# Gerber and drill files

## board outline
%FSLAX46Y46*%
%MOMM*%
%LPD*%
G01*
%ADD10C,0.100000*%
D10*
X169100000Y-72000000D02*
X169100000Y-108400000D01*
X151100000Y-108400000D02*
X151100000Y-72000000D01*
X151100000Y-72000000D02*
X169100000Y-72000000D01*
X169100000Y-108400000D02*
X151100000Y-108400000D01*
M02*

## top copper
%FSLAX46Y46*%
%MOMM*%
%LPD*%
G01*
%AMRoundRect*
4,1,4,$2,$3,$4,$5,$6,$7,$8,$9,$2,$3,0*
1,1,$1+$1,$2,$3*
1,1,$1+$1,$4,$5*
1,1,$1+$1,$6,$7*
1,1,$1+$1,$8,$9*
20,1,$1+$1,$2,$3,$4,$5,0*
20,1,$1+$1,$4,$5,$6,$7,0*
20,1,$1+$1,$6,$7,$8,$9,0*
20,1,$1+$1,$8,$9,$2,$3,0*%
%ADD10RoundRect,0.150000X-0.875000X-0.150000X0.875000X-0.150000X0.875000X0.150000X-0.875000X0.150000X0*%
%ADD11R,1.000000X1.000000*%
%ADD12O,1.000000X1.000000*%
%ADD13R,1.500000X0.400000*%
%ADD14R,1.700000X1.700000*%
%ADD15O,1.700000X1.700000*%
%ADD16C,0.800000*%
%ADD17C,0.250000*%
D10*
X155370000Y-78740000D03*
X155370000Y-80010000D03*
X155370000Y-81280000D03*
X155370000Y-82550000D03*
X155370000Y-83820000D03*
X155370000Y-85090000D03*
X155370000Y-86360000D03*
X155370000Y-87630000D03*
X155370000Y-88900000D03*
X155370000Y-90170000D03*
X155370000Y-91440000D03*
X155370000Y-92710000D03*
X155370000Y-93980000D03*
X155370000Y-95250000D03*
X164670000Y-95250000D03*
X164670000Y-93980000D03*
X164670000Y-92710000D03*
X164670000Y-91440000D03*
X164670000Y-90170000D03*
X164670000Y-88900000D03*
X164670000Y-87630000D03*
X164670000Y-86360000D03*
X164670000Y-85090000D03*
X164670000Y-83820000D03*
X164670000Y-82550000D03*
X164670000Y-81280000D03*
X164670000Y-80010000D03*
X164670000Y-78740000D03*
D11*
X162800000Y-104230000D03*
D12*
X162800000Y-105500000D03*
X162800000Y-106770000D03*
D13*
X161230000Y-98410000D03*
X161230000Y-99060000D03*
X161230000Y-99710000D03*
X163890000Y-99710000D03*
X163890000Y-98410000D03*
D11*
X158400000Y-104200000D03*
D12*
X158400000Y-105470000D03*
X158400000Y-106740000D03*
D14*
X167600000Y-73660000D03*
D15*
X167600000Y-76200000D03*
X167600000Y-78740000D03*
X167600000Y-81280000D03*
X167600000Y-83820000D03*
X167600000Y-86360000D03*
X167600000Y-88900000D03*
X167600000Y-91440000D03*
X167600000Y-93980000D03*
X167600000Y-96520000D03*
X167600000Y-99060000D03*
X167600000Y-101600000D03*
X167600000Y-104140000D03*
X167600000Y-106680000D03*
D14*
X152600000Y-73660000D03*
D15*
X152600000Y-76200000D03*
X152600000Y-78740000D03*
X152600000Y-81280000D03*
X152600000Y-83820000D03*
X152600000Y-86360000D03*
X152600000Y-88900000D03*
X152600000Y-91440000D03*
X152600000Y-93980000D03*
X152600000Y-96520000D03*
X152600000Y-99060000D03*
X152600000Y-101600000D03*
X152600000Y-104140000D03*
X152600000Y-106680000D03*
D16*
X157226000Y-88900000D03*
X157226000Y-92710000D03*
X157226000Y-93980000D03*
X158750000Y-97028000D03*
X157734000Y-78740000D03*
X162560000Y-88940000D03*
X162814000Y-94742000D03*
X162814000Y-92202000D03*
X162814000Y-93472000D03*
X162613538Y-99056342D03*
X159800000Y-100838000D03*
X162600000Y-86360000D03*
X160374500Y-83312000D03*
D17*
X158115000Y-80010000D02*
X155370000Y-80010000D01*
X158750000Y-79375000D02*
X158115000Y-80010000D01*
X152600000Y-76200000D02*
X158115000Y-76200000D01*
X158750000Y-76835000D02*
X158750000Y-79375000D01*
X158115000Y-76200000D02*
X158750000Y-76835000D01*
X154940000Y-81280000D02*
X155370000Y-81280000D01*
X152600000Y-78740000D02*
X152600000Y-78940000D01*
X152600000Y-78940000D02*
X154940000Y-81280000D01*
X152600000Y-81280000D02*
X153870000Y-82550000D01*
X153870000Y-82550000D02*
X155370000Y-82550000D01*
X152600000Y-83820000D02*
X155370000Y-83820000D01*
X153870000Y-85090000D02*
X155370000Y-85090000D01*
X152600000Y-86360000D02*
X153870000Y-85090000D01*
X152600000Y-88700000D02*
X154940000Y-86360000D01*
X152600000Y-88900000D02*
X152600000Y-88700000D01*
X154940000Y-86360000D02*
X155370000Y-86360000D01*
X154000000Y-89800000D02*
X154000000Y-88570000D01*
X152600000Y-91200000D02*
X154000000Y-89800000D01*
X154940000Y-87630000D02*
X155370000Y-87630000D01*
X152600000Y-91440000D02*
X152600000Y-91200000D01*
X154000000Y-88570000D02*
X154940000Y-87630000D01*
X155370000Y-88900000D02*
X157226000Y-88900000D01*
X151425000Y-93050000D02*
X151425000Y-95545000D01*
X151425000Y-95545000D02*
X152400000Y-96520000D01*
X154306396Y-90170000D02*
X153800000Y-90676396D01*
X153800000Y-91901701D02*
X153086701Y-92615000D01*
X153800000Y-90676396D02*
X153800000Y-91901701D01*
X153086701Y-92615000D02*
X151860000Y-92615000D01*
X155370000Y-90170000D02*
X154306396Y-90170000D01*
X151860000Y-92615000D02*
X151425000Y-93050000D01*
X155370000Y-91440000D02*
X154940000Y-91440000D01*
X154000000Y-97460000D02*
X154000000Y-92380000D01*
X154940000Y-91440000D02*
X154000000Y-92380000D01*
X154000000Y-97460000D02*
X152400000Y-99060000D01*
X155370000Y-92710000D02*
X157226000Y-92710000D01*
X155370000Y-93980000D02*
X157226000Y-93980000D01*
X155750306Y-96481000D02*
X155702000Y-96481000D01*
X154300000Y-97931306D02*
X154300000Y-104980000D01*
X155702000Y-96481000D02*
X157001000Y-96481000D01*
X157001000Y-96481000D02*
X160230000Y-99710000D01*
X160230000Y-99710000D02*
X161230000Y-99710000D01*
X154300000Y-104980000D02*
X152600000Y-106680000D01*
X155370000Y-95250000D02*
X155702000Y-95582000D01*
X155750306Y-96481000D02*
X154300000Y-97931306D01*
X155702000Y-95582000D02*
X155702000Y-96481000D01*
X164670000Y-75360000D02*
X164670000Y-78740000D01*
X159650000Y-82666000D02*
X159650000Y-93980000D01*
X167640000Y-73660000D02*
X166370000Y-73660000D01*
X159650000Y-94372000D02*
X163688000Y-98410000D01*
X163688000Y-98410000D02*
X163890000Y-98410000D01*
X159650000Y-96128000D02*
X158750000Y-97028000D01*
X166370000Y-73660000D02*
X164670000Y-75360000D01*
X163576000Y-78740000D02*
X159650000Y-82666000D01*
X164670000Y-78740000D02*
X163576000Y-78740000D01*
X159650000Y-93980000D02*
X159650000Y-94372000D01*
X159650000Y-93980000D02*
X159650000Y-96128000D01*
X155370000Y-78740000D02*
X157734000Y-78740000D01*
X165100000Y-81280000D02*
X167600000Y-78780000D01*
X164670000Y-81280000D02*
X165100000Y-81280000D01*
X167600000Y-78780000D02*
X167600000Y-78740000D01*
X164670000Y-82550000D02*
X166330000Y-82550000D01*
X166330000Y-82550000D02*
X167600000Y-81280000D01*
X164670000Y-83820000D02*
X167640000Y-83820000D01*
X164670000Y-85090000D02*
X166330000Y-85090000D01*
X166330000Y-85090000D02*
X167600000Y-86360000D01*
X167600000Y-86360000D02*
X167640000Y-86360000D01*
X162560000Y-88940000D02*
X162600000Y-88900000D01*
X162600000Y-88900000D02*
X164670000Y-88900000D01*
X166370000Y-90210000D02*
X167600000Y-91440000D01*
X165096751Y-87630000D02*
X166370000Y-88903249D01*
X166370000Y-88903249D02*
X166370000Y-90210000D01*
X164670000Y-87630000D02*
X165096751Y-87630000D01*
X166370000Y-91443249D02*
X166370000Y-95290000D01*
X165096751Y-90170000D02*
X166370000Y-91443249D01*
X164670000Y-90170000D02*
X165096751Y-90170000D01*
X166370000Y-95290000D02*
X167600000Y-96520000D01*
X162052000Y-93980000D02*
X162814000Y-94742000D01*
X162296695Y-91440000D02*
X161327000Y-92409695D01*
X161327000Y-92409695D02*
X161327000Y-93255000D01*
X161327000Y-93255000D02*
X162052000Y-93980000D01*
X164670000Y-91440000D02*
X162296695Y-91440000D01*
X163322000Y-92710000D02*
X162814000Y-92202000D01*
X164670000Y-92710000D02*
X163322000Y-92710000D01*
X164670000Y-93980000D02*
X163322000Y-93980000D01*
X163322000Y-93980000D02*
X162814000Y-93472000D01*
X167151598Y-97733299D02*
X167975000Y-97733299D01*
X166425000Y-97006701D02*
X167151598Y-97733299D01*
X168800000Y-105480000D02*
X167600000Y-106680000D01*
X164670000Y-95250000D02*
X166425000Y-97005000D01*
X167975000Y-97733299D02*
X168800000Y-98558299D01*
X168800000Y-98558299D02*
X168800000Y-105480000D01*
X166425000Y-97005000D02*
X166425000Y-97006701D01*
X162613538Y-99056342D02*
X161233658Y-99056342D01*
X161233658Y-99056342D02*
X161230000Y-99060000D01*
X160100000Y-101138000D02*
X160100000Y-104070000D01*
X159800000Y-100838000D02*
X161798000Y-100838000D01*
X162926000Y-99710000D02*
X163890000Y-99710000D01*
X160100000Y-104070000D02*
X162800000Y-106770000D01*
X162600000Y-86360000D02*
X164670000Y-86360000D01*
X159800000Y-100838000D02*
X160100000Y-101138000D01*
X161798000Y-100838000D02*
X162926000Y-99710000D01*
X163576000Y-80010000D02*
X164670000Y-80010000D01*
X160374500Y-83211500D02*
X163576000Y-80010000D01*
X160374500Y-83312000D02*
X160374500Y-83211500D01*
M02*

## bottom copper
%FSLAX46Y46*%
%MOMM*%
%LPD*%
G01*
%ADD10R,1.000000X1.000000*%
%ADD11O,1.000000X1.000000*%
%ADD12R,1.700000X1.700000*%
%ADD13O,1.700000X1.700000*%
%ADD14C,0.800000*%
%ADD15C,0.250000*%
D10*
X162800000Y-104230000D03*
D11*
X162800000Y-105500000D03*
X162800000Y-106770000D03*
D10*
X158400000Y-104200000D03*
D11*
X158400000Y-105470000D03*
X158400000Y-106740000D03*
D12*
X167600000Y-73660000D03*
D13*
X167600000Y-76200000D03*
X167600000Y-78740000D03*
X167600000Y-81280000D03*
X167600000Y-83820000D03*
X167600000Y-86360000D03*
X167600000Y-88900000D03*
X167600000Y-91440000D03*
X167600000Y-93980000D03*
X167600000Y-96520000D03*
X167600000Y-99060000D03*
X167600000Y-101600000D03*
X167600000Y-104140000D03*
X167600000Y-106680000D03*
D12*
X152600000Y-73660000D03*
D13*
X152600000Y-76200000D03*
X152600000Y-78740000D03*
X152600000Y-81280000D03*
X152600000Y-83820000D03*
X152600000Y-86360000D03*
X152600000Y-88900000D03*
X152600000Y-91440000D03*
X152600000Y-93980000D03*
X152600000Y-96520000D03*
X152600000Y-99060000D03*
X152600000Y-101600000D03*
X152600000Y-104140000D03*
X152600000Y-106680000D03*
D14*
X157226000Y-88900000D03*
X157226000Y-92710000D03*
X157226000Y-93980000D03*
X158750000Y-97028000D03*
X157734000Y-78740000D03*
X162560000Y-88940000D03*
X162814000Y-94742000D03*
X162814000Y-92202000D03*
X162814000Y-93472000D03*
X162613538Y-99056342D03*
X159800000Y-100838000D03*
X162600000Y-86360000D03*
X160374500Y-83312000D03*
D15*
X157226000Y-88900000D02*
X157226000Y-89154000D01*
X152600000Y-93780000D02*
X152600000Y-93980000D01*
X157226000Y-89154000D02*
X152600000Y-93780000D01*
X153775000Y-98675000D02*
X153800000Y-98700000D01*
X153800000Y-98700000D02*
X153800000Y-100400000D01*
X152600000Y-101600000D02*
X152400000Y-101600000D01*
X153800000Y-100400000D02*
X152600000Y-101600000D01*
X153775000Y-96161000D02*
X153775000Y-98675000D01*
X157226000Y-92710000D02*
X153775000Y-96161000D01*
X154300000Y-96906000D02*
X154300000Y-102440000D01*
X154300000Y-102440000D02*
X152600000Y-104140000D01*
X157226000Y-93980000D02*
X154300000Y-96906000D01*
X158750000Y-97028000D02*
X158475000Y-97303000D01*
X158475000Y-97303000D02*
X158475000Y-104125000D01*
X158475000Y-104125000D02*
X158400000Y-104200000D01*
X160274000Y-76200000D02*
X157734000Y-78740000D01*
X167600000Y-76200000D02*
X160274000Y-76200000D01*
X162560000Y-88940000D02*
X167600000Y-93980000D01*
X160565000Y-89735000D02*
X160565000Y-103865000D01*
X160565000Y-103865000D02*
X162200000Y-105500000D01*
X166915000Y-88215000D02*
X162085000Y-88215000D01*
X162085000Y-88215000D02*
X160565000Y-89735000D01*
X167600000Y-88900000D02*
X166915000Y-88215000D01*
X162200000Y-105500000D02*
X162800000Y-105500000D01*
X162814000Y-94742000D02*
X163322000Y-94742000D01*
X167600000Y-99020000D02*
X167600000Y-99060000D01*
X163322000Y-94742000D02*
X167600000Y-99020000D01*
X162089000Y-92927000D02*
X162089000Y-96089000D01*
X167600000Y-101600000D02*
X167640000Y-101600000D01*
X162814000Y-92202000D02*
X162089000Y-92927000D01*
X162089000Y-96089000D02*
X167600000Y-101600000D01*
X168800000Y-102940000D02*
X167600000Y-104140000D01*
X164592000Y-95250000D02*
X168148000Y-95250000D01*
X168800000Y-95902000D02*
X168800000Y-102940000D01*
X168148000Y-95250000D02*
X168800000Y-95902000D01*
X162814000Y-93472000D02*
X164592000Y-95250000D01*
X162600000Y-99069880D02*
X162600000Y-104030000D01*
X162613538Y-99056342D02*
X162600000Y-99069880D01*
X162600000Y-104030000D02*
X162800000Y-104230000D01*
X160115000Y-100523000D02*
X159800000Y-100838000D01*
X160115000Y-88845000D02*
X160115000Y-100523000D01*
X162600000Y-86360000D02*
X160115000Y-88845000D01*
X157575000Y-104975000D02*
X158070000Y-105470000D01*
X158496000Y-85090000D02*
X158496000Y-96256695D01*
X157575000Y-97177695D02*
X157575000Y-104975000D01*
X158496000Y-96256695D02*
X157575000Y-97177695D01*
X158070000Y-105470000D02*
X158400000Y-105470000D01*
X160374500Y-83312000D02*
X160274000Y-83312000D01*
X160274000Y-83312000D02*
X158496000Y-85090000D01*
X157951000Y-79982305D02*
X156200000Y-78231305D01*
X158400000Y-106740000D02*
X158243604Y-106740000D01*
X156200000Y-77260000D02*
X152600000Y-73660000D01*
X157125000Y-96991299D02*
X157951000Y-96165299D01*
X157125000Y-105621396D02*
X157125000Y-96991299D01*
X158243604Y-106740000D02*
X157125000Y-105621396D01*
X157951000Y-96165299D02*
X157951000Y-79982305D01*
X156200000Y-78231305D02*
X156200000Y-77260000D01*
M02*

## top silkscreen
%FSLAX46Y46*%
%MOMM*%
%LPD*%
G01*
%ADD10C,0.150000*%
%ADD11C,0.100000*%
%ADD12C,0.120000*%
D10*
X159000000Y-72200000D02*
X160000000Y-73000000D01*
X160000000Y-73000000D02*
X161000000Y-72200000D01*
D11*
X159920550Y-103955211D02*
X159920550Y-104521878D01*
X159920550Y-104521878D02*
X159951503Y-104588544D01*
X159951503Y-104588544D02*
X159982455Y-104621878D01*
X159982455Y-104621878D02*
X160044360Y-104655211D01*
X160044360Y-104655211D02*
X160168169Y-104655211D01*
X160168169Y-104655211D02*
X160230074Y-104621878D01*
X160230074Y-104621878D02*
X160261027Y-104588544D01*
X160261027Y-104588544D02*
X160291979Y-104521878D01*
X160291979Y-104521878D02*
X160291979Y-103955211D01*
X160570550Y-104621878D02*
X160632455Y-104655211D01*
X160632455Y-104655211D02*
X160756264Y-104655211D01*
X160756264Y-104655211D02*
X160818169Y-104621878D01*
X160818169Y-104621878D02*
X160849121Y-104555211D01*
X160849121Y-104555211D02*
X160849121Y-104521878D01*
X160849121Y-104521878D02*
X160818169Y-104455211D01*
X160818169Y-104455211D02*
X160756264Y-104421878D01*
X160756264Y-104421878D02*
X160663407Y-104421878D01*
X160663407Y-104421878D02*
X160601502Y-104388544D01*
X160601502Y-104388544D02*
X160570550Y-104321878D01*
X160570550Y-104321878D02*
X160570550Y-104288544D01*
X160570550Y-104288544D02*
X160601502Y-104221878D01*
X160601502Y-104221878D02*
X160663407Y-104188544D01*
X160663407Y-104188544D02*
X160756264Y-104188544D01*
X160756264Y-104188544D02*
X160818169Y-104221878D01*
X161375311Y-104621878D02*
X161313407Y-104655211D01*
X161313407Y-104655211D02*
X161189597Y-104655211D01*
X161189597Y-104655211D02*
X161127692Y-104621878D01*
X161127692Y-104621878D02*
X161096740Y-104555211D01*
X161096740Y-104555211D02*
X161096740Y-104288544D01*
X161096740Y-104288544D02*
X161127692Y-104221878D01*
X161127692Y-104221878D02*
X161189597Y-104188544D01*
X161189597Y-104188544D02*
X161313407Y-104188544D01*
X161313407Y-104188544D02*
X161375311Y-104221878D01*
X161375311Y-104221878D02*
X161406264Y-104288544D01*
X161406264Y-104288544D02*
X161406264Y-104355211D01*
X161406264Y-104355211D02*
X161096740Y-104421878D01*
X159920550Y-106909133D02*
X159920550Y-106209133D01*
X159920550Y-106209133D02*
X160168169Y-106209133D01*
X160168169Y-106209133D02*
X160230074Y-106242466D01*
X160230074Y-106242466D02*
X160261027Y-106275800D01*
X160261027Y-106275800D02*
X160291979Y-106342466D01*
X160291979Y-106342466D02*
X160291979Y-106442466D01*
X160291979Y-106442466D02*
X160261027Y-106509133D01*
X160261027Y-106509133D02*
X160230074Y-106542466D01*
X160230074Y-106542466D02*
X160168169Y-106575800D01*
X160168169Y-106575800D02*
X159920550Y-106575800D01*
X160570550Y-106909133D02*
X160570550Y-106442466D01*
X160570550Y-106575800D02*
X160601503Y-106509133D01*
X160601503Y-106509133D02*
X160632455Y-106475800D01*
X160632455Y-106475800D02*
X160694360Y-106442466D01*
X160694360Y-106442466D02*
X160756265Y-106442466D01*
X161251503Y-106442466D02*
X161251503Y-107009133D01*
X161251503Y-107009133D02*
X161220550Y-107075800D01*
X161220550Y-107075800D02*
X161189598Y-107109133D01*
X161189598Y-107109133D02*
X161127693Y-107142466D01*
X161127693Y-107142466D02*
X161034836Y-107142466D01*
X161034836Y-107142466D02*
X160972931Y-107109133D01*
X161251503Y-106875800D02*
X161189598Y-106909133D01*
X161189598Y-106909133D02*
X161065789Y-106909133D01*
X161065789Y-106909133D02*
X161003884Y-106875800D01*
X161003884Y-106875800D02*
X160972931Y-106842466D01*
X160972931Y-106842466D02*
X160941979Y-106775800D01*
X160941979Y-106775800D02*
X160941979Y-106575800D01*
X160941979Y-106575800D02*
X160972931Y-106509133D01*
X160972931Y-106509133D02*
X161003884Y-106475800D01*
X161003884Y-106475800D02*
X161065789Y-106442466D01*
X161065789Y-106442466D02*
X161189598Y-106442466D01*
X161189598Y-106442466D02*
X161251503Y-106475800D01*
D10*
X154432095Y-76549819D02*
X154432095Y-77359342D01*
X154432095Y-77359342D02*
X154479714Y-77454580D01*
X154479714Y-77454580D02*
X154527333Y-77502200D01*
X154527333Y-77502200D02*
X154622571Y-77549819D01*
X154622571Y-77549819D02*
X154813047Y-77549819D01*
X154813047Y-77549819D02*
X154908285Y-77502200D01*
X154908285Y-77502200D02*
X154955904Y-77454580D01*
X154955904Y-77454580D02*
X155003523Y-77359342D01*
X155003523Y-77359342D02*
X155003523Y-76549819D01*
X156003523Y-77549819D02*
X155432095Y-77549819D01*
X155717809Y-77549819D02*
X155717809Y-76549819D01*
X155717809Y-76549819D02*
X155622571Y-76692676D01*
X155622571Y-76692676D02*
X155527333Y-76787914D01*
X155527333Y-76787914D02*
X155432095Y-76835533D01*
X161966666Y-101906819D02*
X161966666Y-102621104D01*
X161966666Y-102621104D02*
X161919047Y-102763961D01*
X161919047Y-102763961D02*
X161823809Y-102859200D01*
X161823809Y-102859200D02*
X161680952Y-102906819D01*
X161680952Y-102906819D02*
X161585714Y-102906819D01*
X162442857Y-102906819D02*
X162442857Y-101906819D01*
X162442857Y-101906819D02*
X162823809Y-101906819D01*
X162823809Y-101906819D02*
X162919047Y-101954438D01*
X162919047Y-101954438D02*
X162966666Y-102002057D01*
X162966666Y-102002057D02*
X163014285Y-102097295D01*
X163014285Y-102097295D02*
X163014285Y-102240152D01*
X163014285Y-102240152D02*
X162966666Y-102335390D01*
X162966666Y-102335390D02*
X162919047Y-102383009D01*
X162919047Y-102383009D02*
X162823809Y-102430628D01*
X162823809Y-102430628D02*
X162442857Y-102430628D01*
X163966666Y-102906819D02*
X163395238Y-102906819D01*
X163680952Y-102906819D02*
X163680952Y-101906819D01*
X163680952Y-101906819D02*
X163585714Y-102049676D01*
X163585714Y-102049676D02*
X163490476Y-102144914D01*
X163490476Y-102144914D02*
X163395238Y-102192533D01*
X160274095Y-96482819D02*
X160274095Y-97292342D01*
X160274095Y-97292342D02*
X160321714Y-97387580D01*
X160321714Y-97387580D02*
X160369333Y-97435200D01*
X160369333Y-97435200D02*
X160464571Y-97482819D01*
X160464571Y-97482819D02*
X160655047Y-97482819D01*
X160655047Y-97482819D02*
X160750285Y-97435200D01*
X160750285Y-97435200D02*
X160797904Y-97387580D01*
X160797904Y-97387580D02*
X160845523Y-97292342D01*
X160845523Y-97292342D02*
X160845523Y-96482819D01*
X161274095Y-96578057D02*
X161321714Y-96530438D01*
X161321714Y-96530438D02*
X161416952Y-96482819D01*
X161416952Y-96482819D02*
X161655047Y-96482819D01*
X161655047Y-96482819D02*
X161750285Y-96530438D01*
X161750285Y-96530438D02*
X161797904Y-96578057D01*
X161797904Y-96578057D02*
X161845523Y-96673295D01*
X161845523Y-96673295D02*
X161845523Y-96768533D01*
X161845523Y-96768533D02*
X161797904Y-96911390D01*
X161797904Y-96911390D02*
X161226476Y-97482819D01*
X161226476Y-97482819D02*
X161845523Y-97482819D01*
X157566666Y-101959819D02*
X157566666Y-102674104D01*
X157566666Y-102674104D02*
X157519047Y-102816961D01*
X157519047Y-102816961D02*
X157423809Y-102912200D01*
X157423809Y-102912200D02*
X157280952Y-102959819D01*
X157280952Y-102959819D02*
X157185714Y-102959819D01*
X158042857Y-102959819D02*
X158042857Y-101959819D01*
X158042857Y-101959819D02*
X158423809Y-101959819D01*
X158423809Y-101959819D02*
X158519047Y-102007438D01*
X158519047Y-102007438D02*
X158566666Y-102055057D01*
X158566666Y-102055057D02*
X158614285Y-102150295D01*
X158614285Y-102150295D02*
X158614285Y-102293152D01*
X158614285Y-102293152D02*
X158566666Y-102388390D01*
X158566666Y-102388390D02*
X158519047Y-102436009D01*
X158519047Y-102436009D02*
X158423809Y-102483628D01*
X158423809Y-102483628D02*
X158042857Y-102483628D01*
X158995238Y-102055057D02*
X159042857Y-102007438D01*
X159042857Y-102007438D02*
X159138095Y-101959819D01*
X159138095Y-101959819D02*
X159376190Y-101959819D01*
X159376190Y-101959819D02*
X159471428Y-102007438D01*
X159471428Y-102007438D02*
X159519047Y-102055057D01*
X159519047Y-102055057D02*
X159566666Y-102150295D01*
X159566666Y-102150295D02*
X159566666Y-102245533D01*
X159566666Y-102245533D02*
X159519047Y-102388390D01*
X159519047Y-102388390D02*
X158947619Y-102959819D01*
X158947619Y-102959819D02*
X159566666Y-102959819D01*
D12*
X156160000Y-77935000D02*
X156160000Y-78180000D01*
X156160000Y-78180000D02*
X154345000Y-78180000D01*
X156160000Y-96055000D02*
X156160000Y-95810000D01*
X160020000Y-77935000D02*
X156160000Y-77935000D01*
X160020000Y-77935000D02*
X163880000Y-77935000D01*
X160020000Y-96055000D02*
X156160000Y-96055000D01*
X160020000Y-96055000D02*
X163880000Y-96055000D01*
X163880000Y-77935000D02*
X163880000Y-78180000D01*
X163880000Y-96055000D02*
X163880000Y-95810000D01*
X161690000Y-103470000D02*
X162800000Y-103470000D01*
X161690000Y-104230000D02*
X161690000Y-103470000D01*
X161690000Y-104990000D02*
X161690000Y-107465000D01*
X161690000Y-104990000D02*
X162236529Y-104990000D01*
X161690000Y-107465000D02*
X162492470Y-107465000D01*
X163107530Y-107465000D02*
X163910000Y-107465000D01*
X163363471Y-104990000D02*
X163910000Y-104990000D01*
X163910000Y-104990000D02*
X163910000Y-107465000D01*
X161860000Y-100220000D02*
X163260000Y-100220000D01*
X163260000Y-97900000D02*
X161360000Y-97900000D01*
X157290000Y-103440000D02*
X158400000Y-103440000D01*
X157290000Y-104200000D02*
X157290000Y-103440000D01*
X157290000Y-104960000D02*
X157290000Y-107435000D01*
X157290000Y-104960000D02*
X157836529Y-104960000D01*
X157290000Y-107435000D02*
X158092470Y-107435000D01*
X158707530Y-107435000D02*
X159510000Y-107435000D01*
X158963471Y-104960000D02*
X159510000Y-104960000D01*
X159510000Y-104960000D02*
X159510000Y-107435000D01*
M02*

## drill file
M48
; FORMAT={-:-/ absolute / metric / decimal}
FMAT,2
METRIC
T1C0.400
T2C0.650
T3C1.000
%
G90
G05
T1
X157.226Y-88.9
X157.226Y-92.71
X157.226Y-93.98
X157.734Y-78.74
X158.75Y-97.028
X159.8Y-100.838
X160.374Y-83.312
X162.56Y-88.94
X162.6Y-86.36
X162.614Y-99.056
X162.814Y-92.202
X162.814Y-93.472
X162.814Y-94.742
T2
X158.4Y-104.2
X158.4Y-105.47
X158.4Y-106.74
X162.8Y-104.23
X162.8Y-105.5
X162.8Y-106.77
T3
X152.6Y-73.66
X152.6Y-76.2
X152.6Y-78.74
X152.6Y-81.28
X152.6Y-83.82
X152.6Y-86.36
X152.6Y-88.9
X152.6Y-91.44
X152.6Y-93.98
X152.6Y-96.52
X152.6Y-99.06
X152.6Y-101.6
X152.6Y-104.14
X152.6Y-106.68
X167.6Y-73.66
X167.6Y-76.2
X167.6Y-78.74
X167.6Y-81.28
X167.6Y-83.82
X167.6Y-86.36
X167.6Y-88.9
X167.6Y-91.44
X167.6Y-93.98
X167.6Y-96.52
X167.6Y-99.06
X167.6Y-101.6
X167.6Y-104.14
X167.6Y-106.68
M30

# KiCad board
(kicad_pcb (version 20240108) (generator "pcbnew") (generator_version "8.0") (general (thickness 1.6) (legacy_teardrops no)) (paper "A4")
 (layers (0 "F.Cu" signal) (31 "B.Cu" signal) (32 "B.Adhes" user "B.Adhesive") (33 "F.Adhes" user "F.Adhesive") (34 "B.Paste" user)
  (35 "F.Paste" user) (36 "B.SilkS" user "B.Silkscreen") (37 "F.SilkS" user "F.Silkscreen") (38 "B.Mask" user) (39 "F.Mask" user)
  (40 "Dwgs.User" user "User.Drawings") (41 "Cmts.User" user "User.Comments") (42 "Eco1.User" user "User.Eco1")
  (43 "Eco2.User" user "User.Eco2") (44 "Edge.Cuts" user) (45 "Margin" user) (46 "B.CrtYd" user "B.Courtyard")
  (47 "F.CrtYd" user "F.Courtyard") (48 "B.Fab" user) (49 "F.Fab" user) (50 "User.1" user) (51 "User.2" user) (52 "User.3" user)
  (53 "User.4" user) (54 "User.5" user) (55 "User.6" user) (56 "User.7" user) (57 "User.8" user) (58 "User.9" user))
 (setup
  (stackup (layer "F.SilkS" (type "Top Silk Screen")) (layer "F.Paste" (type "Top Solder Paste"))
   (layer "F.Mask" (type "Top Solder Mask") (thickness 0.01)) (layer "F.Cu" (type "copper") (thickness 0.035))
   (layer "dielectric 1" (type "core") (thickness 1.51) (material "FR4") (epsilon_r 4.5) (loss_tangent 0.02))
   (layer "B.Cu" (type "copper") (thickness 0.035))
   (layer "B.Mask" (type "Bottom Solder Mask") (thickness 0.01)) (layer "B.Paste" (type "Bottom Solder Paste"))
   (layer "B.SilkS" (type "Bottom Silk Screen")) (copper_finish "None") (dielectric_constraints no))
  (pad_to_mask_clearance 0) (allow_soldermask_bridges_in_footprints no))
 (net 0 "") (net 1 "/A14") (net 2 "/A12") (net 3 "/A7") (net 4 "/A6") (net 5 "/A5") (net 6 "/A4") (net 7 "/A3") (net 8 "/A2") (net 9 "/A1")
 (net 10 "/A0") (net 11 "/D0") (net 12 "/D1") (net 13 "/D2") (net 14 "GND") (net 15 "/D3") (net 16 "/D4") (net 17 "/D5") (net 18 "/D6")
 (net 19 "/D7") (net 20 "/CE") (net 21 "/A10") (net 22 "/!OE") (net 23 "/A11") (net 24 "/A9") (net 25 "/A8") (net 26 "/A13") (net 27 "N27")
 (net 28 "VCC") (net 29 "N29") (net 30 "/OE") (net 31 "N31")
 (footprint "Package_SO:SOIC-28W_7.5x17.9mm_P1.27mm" (layer "F.Cu") (at 160.02 86.995)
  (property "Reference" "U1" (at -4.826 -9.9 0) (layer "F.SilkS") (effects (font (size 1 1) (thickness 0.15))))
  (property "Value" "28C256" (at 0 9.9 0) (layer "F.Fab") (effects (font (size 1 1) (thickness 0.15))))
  (fp_line (start -3.86 -9.06) (end -3.86 -8.815) (stroke (width 0.12) (type solid)) (layer "F.SilkS"))
  (fp_line (start -3.86 -8.815) (end -5.675 -8.815) (stroke (width 0.12) (type solid)) (layer "F.SilkS"))
  (fp_line (start -3.86 9.06) (end -3.86 8.815) (stroke (width 0.12) (type solid)) (layer "F.SilkS"))
  (fp_line (start 0 -9.06) (end -3.86 -9.06) (stroke (width 0.12) (type solid)) (layer "F.SilkS"))
  (fp_line (start 0 -9.06) (end 3.86 -9.06) (stroke (width 0.12) (type solid)) (layer "F.SilkS"))
  (fp_line (start 0 9.06) (end -3.86 9.06) (stroke (width 0.12) (type solid)) (layer "F.SilkS"))
  (fp_line (start 0 9.06) (end 3.86 9.06) (stroke (width 0.12) (type solid)) (layer "F.SilkS"))
  (fp_line (start 3.86 -9.06) (end 3.86 -8.815) (stroke (width 0.12) (type solid)) (layer "F.SilkS"))
  (fp_line (start 3.86 9.06) (end 3.86 8.815) (stroke (width 0.12) (type solid)) (layer "F.SilkS"))
  (pad "1" smd roundrect (at -4.65 -8.255) (size 2.05 0.6) (layers "F.Cu" "F.Paste" "F.Mask") (roundrect_rratio 0.25) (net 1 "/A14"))
  (pad "2" smd roundrect (at -4.65 -6.985) (size 2.05 0.6) (layers "F.Cu" "F.Paste" "F.Mask") (roundrect_rratio 0.25) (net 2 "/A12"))
  (pad "3" smd roundrect (at -4.65 -5.715) (size 2.05 0.6) (layers "F.Cu" "F.Paste" "F.Mask") (roundrect_rratio 0.25) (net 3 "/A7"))
  (pad "4" smd roundrect (at -4.65 -4.445) (size 2.05 0.6) (layers "F.Cu" "F.Paste" "F.Mask") (roundrect_rratio 0.25) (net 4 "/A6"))
  (pad "5" smd roundrect (at -4.65 -3.175) (size 2.05 0.6) (layers "F.Cu" "F.Paste" "F.Mask") (roundrect_rratio 0.25) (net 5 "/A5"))
  (pad "6" smd roundrect (at -4.65 -1.905) (size 2.05 0.6) (layers "F.Cu" "F.Paste" "F.Mask") (roundrect_rratio 0.25) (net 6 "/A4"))
  (pad "7" smd roundrect (at -4.65 -0.635) (size 2.05 0.6) (layers "F.Cu" "F.Paste" "F.Mask") (roundrect_rratio 0.25) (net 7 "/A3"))
  (pad "8" smd roundrect (at -4.65 0.635) (size 2.05 0.6) (layers "F.Cu" "F.Paste" "F.Mask") (roundrect_rratio 0.25) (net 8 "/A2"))
  (pad "9" smd roundrect (at -4.65 1.905) (size 2.05 0.6) (layers "F.Cu" "F.Paste" "F.Mask") (roundrect_rratio 0.25) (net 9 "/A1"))
  (pad "10" smd roundrect (at -4.65 3.175) (size 2.05 0.6) (layers "F.Cu" "F.Paste" "F.Mask") (roundrect_rratio 0.25) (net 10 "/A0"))
  (pad "11" smd roundrect (at -4.65 4.445) (size 2.05 0.6) (layers "F.Cu" "F.Paste" "F.Mask") (roundrect_rratio 0.25) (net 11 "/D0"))
  (pad "12" smd roundrect (at -4.65 5.715) (size 2.05 0.6) (layers "F.Cu" "F.Paste" "F.Mask") (roundrect_rratio 0.25) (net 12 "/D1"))
  (pad "13" smd roundrect (at -4.65 6.985) (size 2.05 0.6) (layers "F.Cu" "F.Paste" "F.Mask") (roundrect_rratio 0.25) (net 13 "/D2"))
  (pad "14" smd roundrect (at -4.65 8.255) (size 2.05 0.6) (layers "F.Cu" "F.Paste" "F.Mask") (roundrect_rratio 0.25) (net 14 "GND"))
  (pad "15" smd roundrect (at 4.65 8.255) (size 2.05 0.6) (layers "F.Cu" "F.Paste" "F.Mask") (roundrect_rratio 0.25) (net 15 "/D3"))
  (pad "16" smd roundrect (at 4.65 6.985) (size 2.05 0.6) (layers "F.Cu" "F.Paste" "F.Mask") (roundrect_rratio 0.25) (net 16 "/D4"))
  (pad "17" smd roundrect (at 4.65 5.715) (size 2.05 0.6) (layers "F.Cu" "F.Paste" "F.Mask") (roundrect_rratio 0.25) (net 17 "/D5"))
  (pad "18" smd roundrect (at 4.65 4.445) (size 2.05 0.6) (layers "F.Cu" "F.Paste" "F.Mask") (roundrect_rratio 0.25) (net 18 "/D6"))
  (pad "19" smd roundrect (at 4.65 3.175) (size 2.05 0.6) (layers "F.Cu" "F.Paste" "F.Mask") (roundrect_rratio 0.25) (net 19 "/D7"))
  (pad "20" smd roundrect (at 4.65 1.905) (size 2.05 0.6) (layers "F.Cu" "F.Paste" "F.Mask") (roundrect_rratio 0.25) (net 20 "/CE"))
  (pad "21" smd roundrect (at 4.65 0.635) (size 2.05 0.6) (layers "F.Cu" "F.Paste" "F.Mask") (roundrect_rratio 0.25) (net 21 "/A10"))
  (pad "22" smd roundrect (at 4.65 -0.635) (size 2.05 0.6) (layers "F.Cu" "F.Paste" "F.Mask") (roundrect_rratio 0.25) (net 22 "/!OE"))
  (pad "23" smd roundrect (at 4.65 -1.905) (size 2.05 0.6) (layers "F.Cu" "F.Paste" "F.Mask") (roundrect_rratio 0.25) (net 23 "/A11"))
  (pad "24" smd roundrect (at 4.65 -3.175) (size 2.05 0.6) (layers "F.Cu" "F.Paste" "F.Mask") (roundrect_rratio 0.25) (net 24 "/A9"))
  (pad "25" smd roundrect (at 4.65 -4.445) (size 2.05 0.6) (layers "F.Cu" "F.Paste" "F.Mask") (roundrect_rratio 0.25) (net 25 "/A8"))
  (pad "26" smd roundrect (at 4.65 -5.715) (size 2.05 0.6) (layers "F.Cu" "F.Paste" "F.Mask") (roundrect_rratio 0.25) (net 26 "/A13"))
  (pad "27" smd roundrect (at 4.65 -6.985) (size 2.05 0.6) (layers "F.Cu" "F.Paste" "F.Mask") (roundrect_rratio 0.25) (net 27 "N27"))
  (pad "28" smd roundrect (at 4.65 -8.255) (size 2.05 0.6) (layers "F.Cu" "F.Paste" "F.Mask") (roundrect_rratio 0.25) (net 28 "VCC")))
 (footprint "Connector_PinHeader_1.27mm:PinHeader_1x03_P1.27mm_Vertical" (layer "F.Cu") (at 162.8 104.23)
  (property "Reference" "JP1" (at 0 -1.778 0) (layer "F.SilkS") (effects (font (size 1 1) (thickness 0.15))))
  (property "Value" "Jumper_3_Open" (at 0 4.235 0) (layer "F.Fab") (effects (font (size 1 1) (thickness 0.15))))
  (fp_line (start -1.11 -0.76) (end 0 -0.76) (stroke (width 0.12) (type solid)) (layer "F.SilkS"))
  (fp_line (start -1.11 0) (end -1.11 -0.76) (stroke (width 0.12) (type solid)) (layer "F.SilkS"))
  (fp_line (start -1.11 0.76) (end -1.11 3.235) (stroke (width 0.12) (type solid)) (layer "F.SilkS"))
  (fp_line (start -1.11 0.76) (end -0.563471 0.76) (stroke (width 0.12) (type solid)) (layer "F.SilkS"))
  (fp_line (start -1.11 3.235) (end -0.30753 3.235) (stroke (width 0.12) (type solid)) (layer "F.SilkS"))
  (fp_line (start 0.30753 3.235) (end 1.11 3.235) (stroke (width 0.12) (type solid)) (layer "F.SilkS"))
  (fp_line (start 0.563471 0.76) (end 1.11 0.76) (stroke (width 0.12) (type solid)) (layer "F.SilkS"))
  (fp_line (start 1.11 0.76) (end 1.11 3.235) (stroke (width 0.12) (type solid)) (layer "F.SilkS"))
  (pad "1" thru_hole rect (at 0 0) (size 1 1) (drill 0.65) (layers "*.Cu" "*.Mask") (remove_unused_layers no) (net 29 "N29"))
  (pad "2" thru_hole oval (at 0 1.27) (size 1 1) (drill 0.65) (layers "*.Cu" "*.Mask") (remove_unused_layers no) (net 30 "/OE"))
  (pad "3" thru_hole oval (at 0 2.54) (size 1 1) (drill 0.65) (layers "*.Cu" "*.Mask") (remove_unused_layers no) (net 22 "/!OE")))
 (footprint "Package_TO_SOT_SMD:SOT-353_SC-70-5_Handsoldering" (layer "F.Cu") (at 162.56 99.06)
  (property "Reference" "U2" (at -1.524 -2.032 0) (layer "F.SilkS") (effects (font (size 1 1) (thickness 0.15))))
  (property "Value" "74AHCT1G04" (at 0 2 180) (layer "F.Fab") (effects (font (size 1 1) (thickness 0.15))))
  (fp_line (start -0.7 1.16) (end 0.7 1.16) (stroke (width 0.12) (type solid)) (layer "F.SilkS"))
  (fp_line (start 0.7 -1.16) (end -1.2 -1.16) (stroke (width 0.12) (type solid)) (layer "F.SilkS"))
  (pad "1" smd rect (at -1.33 -0.65) (size 1.5 0.4) (layers "F.Cu" "F.Paste" "F.Mask"))
  (pad "2" smd rect (at -1.33 0) (size 1.5 0.4) (layers "F.Cu" "F.Paste" "F.Mask") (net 29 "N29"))
  (pad "3" smd rect (at -1.33 0.65) (size 1.5 0.4) (layers "F.Cu" "F.Paste" "F.Mask") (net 14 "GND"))
  (pad "4" smd rect (at 1.33 0.65) (size 1.5 0.4) (layers "F.Cu" "F.Paste" "F.Mask") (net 22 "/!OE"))
  (pad "5" smd rect (at 1.33 -0.65) (size 1.5 0.4) (layers "F.Cu" "F.Paste" "F.Mask") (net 28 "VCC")))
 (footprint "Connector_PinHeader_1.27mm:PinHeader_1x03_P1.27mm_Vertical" (layer "F.Cu") (at 158.4 104.2)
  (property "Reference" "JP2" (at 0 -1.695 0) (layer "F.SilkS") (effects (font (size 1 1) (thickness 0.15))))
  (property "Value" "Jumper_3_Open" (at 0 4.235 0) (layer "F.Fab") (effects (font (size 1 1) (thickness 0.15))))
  (fp_line (start -1.11 -0.76) (end 0 -0.76) (stroke (width 0.12) (type solid)) (layer "F.SilkS"))
  (fp_line (start -1.11 0) (end -1.11 -0.76) (stroke (width 0.12) (type solid)) (layer "F.SilkS"))
  (fp_line (start -1.11 0.76) (end -1.11 3.235) (stroke (width 0.12) (type solid)) (layer "F.SilkS"))
  (fp_line (start -1.11 0.76) (end -0.563471 0.76) (stroke (width 0.12) (type solid)) (layer "F.SilkS"))
  (fp_line (start -1.11 3.235) (end -0.30753 3.235) (stroke (width 0.12) (type solid)) (layer "F.SilkS"))
  (fp_line (start 0.30753 3.235) (end 1.11 3.235) (stroke (width 0.12) (type solid)) (layer "F.SilkS"))
  (fp_line (start 0.563471 0.76) (end 1.11 0.76) (stroke (width 0.12) (type solid)) (layer "F.SilkS"))
  (fp_line (start 1.11 0.76) (end 1.11 3.235) (stroke (width 0.12) (type solid)) (layer "F.SilkS"))
  (pad "1" thru_hole rect (at 0 0) (size 1 1) (drill 0.65) (layers "*.Cu" "*.Mask") (remove_unused_layers no) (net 28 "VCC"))
  (pad "2" thru_hole oval (at 0 1.27) (size 1 1) (drill 0.65) (layers "*.Cu" "*.Mask") (remove_unused_layers no) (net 27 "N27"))
  (pad "3" thru_hole oval (at 0 2.54) (size 1 1) (drill 0.65) (layers "*.Cu" "*.Mask") (remove_unused_layers no) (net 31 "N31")))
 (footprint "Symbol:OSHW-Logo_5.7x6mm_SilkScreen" (layer "B.Cu") (at 159.893 77.336 180)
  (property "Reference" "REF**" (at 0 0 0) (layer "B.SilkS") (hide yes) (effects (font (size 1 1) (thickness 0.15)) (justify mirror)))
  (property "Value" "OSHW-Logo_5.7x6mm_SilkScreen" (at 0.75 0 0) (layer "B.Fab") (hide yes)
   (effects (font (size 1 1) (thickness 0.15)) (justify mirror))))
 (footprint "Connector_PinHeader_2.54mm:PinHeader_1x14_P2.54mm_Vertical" (layer "B.Cu") (at 167.6 73.66 180)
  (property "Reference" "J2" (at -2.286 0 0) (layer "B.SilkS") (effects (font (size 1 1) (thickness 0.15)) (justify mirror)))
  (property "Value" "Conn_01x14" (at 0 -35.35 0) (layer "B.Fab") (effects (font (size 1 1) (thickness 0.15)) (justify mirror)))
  (pad "1" thru_hole rect (at 0 0 180) (size 1.7 1.7) (drill 1) (layers "*.Cu" "*.Mask") (remove_unused_layers no) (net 28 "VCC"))
  (pad "2" thru_hole oval (at 0 -2.54 180) (size 1.7 1.7) (drill 1) (layers "*.Cu" "*.Mask") (remove_unused_layers no) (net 1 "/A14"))
  (pad "3" thru_hole oval (at 0 -5.08 180) (size 1.7 1.7) (drill 1) (layers "*.Cu" "*.Mask") (remove_unused_layers no) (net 26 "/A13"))
  (pad "4" thru_hole oval (at 0 -7.62 180) (size 1.7 1.7) (drill 1) (layers "*.Cu" "*.Mask") (remove_unused_layers no) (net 25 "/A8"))
  (pad "5" thru_hole oval (at 0 -10.16 180) (size 1.7 1.7) (drill 1) (layers "*.Cu" "*.Mask") (remove_unused_layers no) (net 24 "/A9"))
  (pad "6" thru_hole oval (at 0 -12.7 180) (size 1.7 1.7) (drill 1) (layers "*.Cu" "*.Mask") (remove_unused_layers no) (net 23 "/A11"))
  (pad "7" thru_hole oval (at 0 -15.24 180) (size 1.7 1.7) (drill 1) (layers "*.Cu" "*.Mask") (remove_unused_layers no) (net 30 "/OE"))
  (pad "8" thru_hole oval (at 0 -17.78 180) (size 1.7 1.7) (drill 1) (layers "*.Cu" "*.Mask") (remove_unused_layers no) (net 21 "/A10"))
  (pad "9" thru_hole oval (at 0 -20.32 180) (size 1.7 1.7) (drill 1) (layers "*.Cu" "*.Mask") (remove_unused_layers no) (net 20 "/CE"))
  (pad "10" thru_hole oval (at 0 -22.86 180) (size 1.7 1.7) (drill 1) (layers "*.Cu" "*.Mask") (remove_unused_layers no) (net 19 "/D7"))
  (pad "11" thru_hole oval (at 0 -25.4 180) (size 1.7 1.7) (drill 1) (layers "*.Cu" "*.Mask") (remove_unused_layers no) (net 18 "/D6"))
  (pad "12" thru_hole oval (at 0 -27.94 180) (size 1.7 1.7) (drill 1) (layers "*.Cu" "*.Mask") (remove_unused_layers no) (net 17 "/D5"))
  (pad "13" thru_hole oval (at 0 -30.48 180) (size 1.7 1.7) (drill 1) (layers "*.Cu" "*.Mask") (remove_unused_layers no) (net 16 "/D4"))
  (pad "14" thru_hole oval (at 0 -33.02 180) (size 1.7 1.7) (drill 1) (layers "*.Cu" "*.Mask") (remove_unused_layers no) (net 15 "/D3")))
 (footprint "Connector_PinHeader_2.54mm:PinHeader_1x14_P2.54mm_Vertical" (layer "B.Cu") (at 152.6 73.66 180)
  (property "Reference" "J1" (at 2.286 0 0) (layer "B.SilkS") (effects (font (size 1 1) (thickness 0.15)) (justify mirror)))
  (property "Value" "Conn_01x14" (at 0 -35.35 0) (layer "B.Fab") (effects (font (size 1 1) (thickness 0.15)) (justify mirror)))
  (pad "1" thru_hole rect (at 0 0 180) (size 1.7 1.7) (drill 1) (layers "*.Cu" "*.Mask") (remove_unused_layers no) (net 31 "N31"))
  (pad "2" thru_hole oval (at 0 -2.54 180) (size 1.7 1.7) (drill 1) (layers "*.Cu" "*.Mask") (remove_unused_layers no) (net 2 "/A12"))
  (pad "3" thru_hole oval (at 0 -5.08 180) (size 1.7 1.7) (drill 1) (layers "*.Cu" "*.Mask") (remove_unused_layers no) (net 3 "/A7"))
  (pad "4" thru_hole oval (at 0 -7.62 180) (size 1.7 1.7) (drill 1) (layers "*.Cu" "*.Mask") (remove_unused_layers no) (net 4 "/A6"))
  (pad "5" thru_hole oval (at 0 -10.16 180) (size 1.7 1.7) (drill 1) (layers "*.Cu" "*.Mask") (remove_unused_layers no) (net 5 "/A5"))
  (pad "6" thru_hole oval (at 0 -12.7 180) (size 1.7 1.7) (drill 1) (layers "*.Cu" "*.Mask") (remove_unused_layers no) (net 6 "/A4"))
  (pad "7" thru_hole oval (at 0 -15.24 180) (size 1.7 1.7) (drill 1) (layers "*.Cu" "*.Mask") (remove_unused_layers no) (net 7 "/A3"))
  (pad "8" thru_hole oval (at 0 -17.78 180) (size 1.7 1.7) (drill 1) (layers "*.Cu" "*.Mask") (remove_unused_layers no) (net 8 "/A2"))
  (pad "9" thru_hole oval (at 0 -20.32 180) (size 1.7 1.7) (drill 1) (layers "*.Cu" "*.Mask") (remove_unused_layers no) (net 9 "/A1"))
  (pad "10" thru_hole oval (at 0 -22.86 180) (size 1.7 1.7) (drill 1) (layers "*.Cu" "*.Mask") (remove_unused_layers no) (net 10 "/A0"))
  (pad "11" thru_hole oval (at 0 -25.4 180) (size 1.7 1.7) (drill 1) (layers "*.Cu" "*.Mask") (remove_unused_layers no) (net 11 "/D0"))
  (pad "12" thru_hole oval (at 0 -27.94 180) (size 1.7 1.7) (drill 1) (layers "*.Cu" "*.Mask") (remove_unused_layers no) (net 12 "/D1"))
  (pad "13" thru_hole oval (at 0 -30.48 180) (size 1.7 1.7) (drill 1) (layers "*.Cu" "*.Mask") (remove_unused_layers no) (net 13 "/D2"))
  (pad "14" thru_hole oval (at 0 -33.02 180) (size 1.7 1.7) (drill 1) (layers "*.Cu" "*.Mask") (remove_unused_layers no) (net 14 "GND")))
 (gr_line (start 159 72.2) (end 160 73) (stroke (width 0.15) (type default)) (layer "F.SilkS"))
 (gr_line (start 160 73) (end 161 72.2) (stroke (width 0.15) (type default)) (layer "F.SilkS"))
 (gr_line (start 169.1 72) (end 169.1 108.4) (stroke (width 0.1) (type default)) (layer "Edge.Cuts"))
 (gr_line (start 151.1 108.4) (end 151.1 72) (stroke (width 0.1) (type default)) (layer "Edge.Cuts"))
 (gr_line (start 151.1 72) (end 169.1 72) (stroke (width 0.1) (type default)) (layer "Edge.Cuts"))
 (gr_line (start 169.1 108.4) (end 151.1 108.4) (stroke (width 0.1) (type default)) (layer "Edge.Cuts"))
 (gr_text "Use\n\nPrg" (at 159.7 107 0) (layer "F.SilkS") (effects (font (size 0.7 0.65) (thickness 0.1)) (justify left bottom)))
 (segment (start 158.115 80.01) (end 155.37 80.01) (width 0.25) (layer "F.Cu") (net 2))
 (segment (start 158.75 79.375) (end 158.115 80.01) (width 0.25) (layer "F.Cu") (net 2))
 (segment (start 152.6 76.2) (end 158.115 76.2) (width 0.25) (layer "F.Cu") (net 2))
 (segment (start 158.75 76.835) (end 158.75 79.375) (width 0.25) (layer "F.Cu") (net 2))
 (segment (start 158.115 76.2) (end 158.75 76.835) (width 0.25) (layer "F.Cu") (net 2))
 (segment (start 154.94 81.28) (end 155.37 81.28) (width 0.25) (layer "F.Cu") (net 3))
 (segment (start 152.6 78.74) (end 152.6 78.94) (width 0.25) (layer "F.Cu") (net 3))
 (segment (start 152.6 78.94) (end 154.94 81.28) (width 0.25) (layer "F.Cu") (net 3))
 (segment (start 152.6 81.28) (end 153.87 82.55) (width 0.25) (layer "F.Cu") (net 4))
 (segment (start 153.87 82.55) (end 155.37 82.55) (width 0.25) (layer "F.Cu") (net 4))
 (segment (start 152.6 83.82) (end 155.37 83.82) (width 0.25) (layer "F.Cu") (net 5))
 (segment (start 153.87 85.09) (end 155.37 85.09) (width 0.25) (layer "F.Cu") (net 6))
 (segment (start 152.6 86.36) (end 153.87 85.09) (width 0.25) (layer "F.Cu") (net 6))
 (segment (start 152.6 88.7) (end 154.94 86.36) (width 0.25) (layer "F.Cu") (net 7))
 (segment (start 152.6 88.9) (end 152.6 88.7) (width 0.25) (layer "F.Cu") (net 7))
 (segment (start 154.94 86.36) (end 155.37 86.36) (width 0.25) (layer "F.Cu") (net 7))
 (segment (start 154 89.8) (end 154 88.57) (width 0.25) (layer "F.Cu") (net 8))
 (segment (start 152.6 91.2) (end 154 89.8) (width 0.25) (layer "F.Cu") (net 8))
 (segment (start 154.94 87.63) (end 155.37 87.63) (width 0.25) (layer "F.Cu") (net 8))
 (segment (start 152.6 91.44) (end 152.6 91.2) (width 0.25) (layer "F.Cu") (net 8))
 (segment (start 154 88.57) (end 154.94 87.63) (width 0.25) (layer "F.Cu") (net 8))
 (segment (start 155.37 88.9) (end 157.226 88.9) (width 0.25) (layer "F.Cu") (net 9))
 (via (at 157.226 88.9) (size 0.8) (drill 0.4) (layers "F.Cu" "B.Cu") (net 9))
 (segment (start 157.226 88.9) (end 157.226 89.154) (width 0.25) (layer "B.Cu") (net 9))
 (segment (start 152.6 93.78) (end 152.6 93.98) (width 0.25) (layer "B.Cu") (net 9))
 (segment (start 157.226 89.154) (end 152.6 93.78) (width 0.25) (layer "B.Cu") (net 9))
 (segment (start 151.425 93.05) (end 151.425 95.545) (width 0.25) (layer "F.Cu") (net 10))
 (segment (start 151.425 95.545) (end 152.4 96.52) (width 0.25) (layer "F.Cu") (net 10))
 (segment (start 154.306396 90.17) (end 153.8 90.676396) (width 0.25) (layer "F.Cu") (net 10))
 (segment (start 153.8 91.901701) (end 153.086701 92.615) (width 0.25) (layer "F.Cu") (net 10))
 (segment (start 153.8 90.676396) (end 153.8 91.901701) (width 0.25) (layer "F.Cu") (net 10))
 (segment (start 153.086701 92.615) (end 151.86 92.615) (width 0.25) (layer "F.Cu") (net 10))
 (segment (start 155.37 90.17) (end 154.306396 90.17) (width 0.25) (layer "F.Cu") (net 10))
 (segment (start 151.86 92.615) (end 151.425 93.05) (width 0.25) (layer "F.Cu") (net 10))
 (segment (start 155.37 91.44) (end 154.94 91.44) (width 0.25) (layer "F.Cu") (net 11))
 (segment (start 154 97.46) (end 154 92.38) (width 0.25) (layer "F.Cu") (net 11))
 (segment (start 154.94 91.44) (end 154 92.38) (width 0.25) (layer "F.Cu") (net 11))
 (segment (start 154 97.46) (end 152.4 99.06) (width 0.25) (layer "F.Cu") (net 11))
 (segment (start 155.37 92.71) (end 157.226 92.71) (width 0.25) (layer "F.Cu") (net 12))
 (via (at 157.226 92.71) (size 0.8) (drill 0.4) (layers "F.Cu" "B.Cu") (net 12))
 (segment (start 153.775 98.675) (end 153.8 98.7) (width 0.25) (layer "B.Cu") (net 12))
 (segment (start 153.8 98.7) (end 153.8 100.4) (width 0.25) (layer "B.Cu") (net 12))
 (segment (start 152.6 101.6) (end 152.4 101.6) (width 0.25) (layer "B.Cu") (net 12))
 (segment (start 153.8 100.4) (end 152.6 101.6) (width 0.25) (layer "B.Cu") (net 12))
 (segment (start 153.775 96.161) (end 153.775 98.675) (width 0.25) (layer "B.Cu") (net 12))
 (segment (start 157.226 92.71) (end 153.775 96.161) (width 0.25) (layer "B.Cu") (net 12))
 (segment (start 155.37 93.98) (end 157.226 93.98) (width 0.25) (layer "F.Cu") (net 13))
 (via (at 157.226 93.98) (size 0.8) (drill 0.4) (layers "F.Cu" "B.Cu") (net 13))
 (segment (start 154.3 96.906) (end 154.3 102.44) (width 0.25) (layer "B.Cu") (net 13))
 (segment (start 154.3 102.44) (end 152.6 104.14) (width 0.25) (layer "B.Cu") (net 13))
 (segment (start 157.226 93.98) (end 154.3 96.906) (width 0.25) (layer "B.Cu") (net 13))
 (segment (start 155.750306 96.481) (end 155.702 96.481) (width 0.25) (layer "F.Cu") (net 14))
 (segment (start 154.3 97.931306) (end 154.3 104.98) (width 0.25) (layer "F.Cu") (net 14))
 (segment (start 155.702 96.481) (end 157.001 96.481) (width 0.25) (layer "F.Cu") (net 14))
 (segment (start 157.001 96.481) (end 160.23 99.71) (width 0.25) (layer "F.Cu") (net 14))
 (segment (start 160.23 99.71) (end 161.23 99.71) (width 0.25) (layer "F.Cu") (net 14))
 (segment (start 154.3 104.98) (end 152.6 106.68) (width 0.25) (layer "F.Cu") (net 14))
 (segment (start 155.37 95.25) (end 155.702 95.582) (width 0.25) (layer "F.Cu") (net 14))
 (segment (start 155.750306 96.481) (end 154.3 97.931306) (width 0.25) (layer "F.Cu") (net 14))
 (segment (start 155.702 95.582) (end 155.702 96.481) (width 0.25) (layer "F.Cu") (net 14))
 (segment (start 164.67 75.36) (end 164.67 78.74) (width 0.25) (layer "F.Cu") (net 28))
 (segment (start 159.65 82.666) (end 159.65 93.98) (width 0.25) (layer "F.Cu") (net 28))
 (segment (start 167.64 73.66) (end 166.37 73.66) (width 0.25) (layer "F.Cu") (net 28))
 (segment (start 159.65 94.372) (end 163.688 98.41) (width 0.25) (layer "F.Cu") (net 28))
 (segment (start 163.688 98.41) (end 163.89 98.41) (width 0.25) (layer "F.Cu") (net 28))
 (segment (start 159.65 96.128) (end 158.75 97.028) (width 0.25) (layer "F.Cu") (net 28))
 (segment (start 166.37 73.66) (end 164.67 75.36) (width 0.25) (layer "F.Cu") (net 28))
 (segment (start 163.576 78.74) (end 159.65 82.666) (width 0.25) (layer "F.Cu") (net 28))
 (segment (start 164.67 78.74) (end 163.576 78.74) (width 0.25) (layer "F.Cu") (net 28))
 (segment (start 159.65 93.98) (end 159.65 94.372) (width 0.25) (layer "F.Cu") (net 28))
 (segment (start 159.65 93.98) (end 159.65 96.128) (width 0.25) (layer "F.Cu") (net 28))
 (via (at 158.75 97.028) (size 0.8) (drill 0.4) (layers "F.Cu" "B.Cu") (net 28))
 (segment (start 158.75 97.028) (end 158.475 97.303) (width 0.25) (layer "B.Cu") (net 28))
 (segment (start 158.475 97.303) (end 158.475 104.125) (width 0.25) (layer "B.Cu") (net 28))
 (segment (start 158.475 104.125) (end 158.4 104.2) (width 0.25) (layer "B.Cu") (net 28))
 (segment (start 155.37 78.74) (end 157.734 78.74) (width 0.25) (layer "F.Cu") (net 1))
 (via (at 157.734 78.74) (size 0.8) (drill 0.4) (layers "F.Cu" "B.Cu") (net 1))
 (segment (start 160.274 76.2) (end 157.734 78.74) (width 0.25) (layer "B.Cu") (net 1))
 (segment (start 167.6 76.2) (end 160.274 76.2) (width 0.25) (layer "B.Cu") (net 1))
 (segment (start 165.1 81.28) (end 167.6 78.78) (width 0.25) (layer "F.Cu") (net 26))
 (segment (start 164.67 81.28) (end 165.1 81.28) (width 0.25) (layer "F.Cu") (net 26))
 (segment (start 167.6 78.78) (end 167.6 78.74) (width 0.25) (layer "F.Cu") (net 26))
 (segment (start 164.67 82.55) (end 166.33 82.55) (width 0.25) (layer "F.Cu") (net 25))
 (segment (start 166.33 82.55) (end 167.6 81.28) (width 0.25) (layer "F.Cu") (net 25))
 (segment (start 164.67 83.82) (end 167.64 83.82) (width 0.25) (layer "F.Cu") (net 24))
 (segment (start 164.67 85.09) (end 166.33 85.09) (width 0.25) (layer "F.Cu") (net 23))
 (segment (start 166.33 85.09) (end 167.6 86.36) (width 0.25) (layer "F.Cu") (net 23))
 (segment (start 167.6 86.36) (end 167.64 86.36) (width 0.25) (layer "F.Cu") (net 23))
 (segment (start 162.56 88.94) (end 162.6 88.9) (width 0.25) (layer "F.Cu") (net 20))
 (segment (start 162.6 88.9) (end 164.67 88.9) (width 0.25) (layer "F.Cu") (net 20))
 (via (at 162.56 88.94) (size 0.8) (drill 0.4) (layers "F.Cu" "B.Cu") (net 20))
 (segment (start 162.56 88.94) (end 167.6 93.98) (width 0.25) (layer "B.Cu") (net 20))
 (segment (start 166.37 90.21) (end 167.6 91.44) (width 0.25) (layer "F.Cu") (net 21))
 (segment (start 165.096751 87.63) (end 166.37 88.903249) (width 0.25) (layer "F.Cu") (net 21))
 (segment (start 166.37 88.903249) (end 166.37 90.21) (width 0.25) (layer "F.Cu") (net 21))
 (segment (start 164.67 87.63) (end 165.096751 87.63) (width 0.25) (layer "F.Cu") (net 21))
 (segment (start 160.565 89.735) (end 160.565 103.865) (width 0.25) (layer "B.Cu") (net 30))
 (segment (start 160.565 103.865) (end 162.2 105.5) (width 0.25) (layer "B.Cu") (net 30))
 (segment (start 166.915 88.215) (end 162.085 88.215) (width 0.25) (layer "B.Cu") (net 30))
 (segment (start 162.085 88.215) (end 160.565 89.735) (width 0.25) (layer "B.Cu") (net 30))
 (segment (start 167.6 88.9) (end 166.915 88.215) (width 0.25) (layer "B.Cu") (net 30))
 (segment (start 162.2 105.5) (end 162.8 105.5) (width 0.25) (layer "B.Cu") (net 30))
 (segment (start 166.37 91.443249) (end 166.37 95.29) (width 0.25) (layer "F.Cu") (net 19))
 (segment (start 165.096751 90.17) (end 166.37 91.443249) (width 0.25) (layer "F.Cu") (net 19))
 (segment (start 164.67 90.17) (end 165.096751 90.17) (width 0.25) (layer "F.Cu") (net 19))
 (segment (start 166.37 95.29) (end 167.6 96.52) (width 0.25) (layer "F.Cu") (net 19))
 (segment (start 162.052 93.98) (end 162.814 94.742) (width 0.25) (layer "F.Cu") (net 18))
 (segment (start 162.296695 91.44) (end 161.327 92.409695) (width 0.25) (layer "F.Cu") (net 18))
 (segment (start 161.327 92.409695) (end 161.327 93.255) (width 0.25) (layer "F.Cu") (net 18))
 (segment (start 161.327 93.255) (end 162.052 93.98) (width 0.25) (layer "F.Cu") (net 18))
 (segment (start 164.67 91.44) (end 162.296695 91.44) (width 0.25) (layer "F.Cu") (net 18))
 (via (at 162.814 94.742) (size 0.8) (drill 0.4) (layers "F.Cu" "B.Cu") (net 18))
 (segment (start 162.814 94.742) (end 163.322 94.742) (width 0.25) (layer "B.Cu") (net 18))
 (segment (start 167.6 99.02) (end 167.6 99.06) (width 0.25) (layer "B.Cu") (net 18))
 (segment (start 163.322 94.742) (end 167.6 99.02) (width 0.25) (layer "B.Cu") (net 18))
 (segment (start 163.322 92.71) (end 162.814 92.202) (width 0.25) (layer "F.Cu") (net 17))
 (segment (start 164.67 92.71) (end 163.322 92.71) (width 0.25) (layer "F.Cu") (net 17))
 (via (at 162.814 92.202) (size 0.8) (drill 0.4) (layers "F.Cu" "B.Cu") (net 17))
 (segment (start 162.089 92.927) (end 162.089 96.089) (width 0.25) (layer "B.Cu") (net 17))
 (segment (start 167.6 101.6) (end 167.64 101.6) (width 0.25) (layer "B.Cu") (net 17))
 (segment (start 162.814 92.202) (end 162.089 92.927) (width 0.25) (layer "B.Cu") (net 17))
 (segment (start 162.089 96.089) (end 167.6 101.6) (width 0.25) (layer "B.Cu") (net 17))
 (segment (start 164.67 93.98) (end 163.322 93.98) (width 0.25) (layer "F.Cu") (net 16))
 (segment (start 163.322 93.98) (end 162.814 93.472) (width 0.25) (layer "F.Cu") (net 16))
 (via (at 162.814 93.472) (size 0.8) (drill 0.4) (layers "F.Cu" "B.Cu") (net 16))
 (segment (start 168.8 102.94) (end 167.6 104.14) (width 0.25) (layer "B.Cu") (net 16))
 (segment (start 164.592 95.25) (end 168.148 95.25) (width 0.25) (layer "B.Cu") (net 16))
 (segment (start 168.8 95.902) (end 168.8 102.94) (width 0.25) (layer "B.Cu") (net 16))
 (segment (start 168.148 95.25) (end 168.8 95.902) (width 0.25) (layer "B.Cu") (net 16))
 (segment (start 162.814 93.472) (end 164.592 95.25) (width 0.25) (layer "B.Cu") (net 16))
 (segment (start 167.151598 97.733299) (end 167.975 97.733299) (width 0.25) (layer "F.Cu") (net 15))
 (segment (start 166.425 97.006701) (end 167.151598 97.733299) (width 0.25) (layer "F.Cu") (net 15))
 (segment (start 168.8 105.48) (end 167.6 106.68) (width 0.25) (layer "F.Cu") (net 15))
 (segment (start 164.67 95.25) (end 166.425 97.005) (width 0.25) (layer "F.Cu") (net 15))
 (segment (start 167.975 97.733299) (end 168.8 98.558299) (width 0.25) (layer "F.Cu") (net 15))
 (segment (start 168.8 98.558299) (end 168.8 105.48) (width 0.25) (layer "F.Cu") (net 15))
 (segment (start 166.425 97.005) (end 166.425 97.006701) (width 0.25) (layer "F.Cu") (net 15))
 (segment (start 162.613538 99.056342) (end 161.233658 99.056342) (width 0.25) (layer "F.Cu") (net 29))
 (segment (start 161.233658 99.056342) (end 161.23 99.06) (width 0.25) (layer "F.Cu") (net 29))
 (via (at 162.613538 99.056342) (size 0.8) (drill 0.4) (layers "F.Cu" "B.Cu") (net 29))
 (segment (start 162.6 99.06988) (end 162.6 104.03) (width 0.25) (layer "B.Cu") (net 29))
 (segment (start 162.613538 99.056342) (end 162.6 99.06988) (width 0.25) (layer "B.Cu") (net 29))
 (segment (start 162.6 104.03) (end 162.8 104.23) (width 0.25) (layer "B.Cu") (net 29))
 (segment (start 160.1 101.138) (end 160.1 104.07) (width 0.25) (layer "F.Cu") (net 22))
 (segment (start 159.8 100.838) (end 161.798 100.838) (width 0.25) (layer "F.Cu") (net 22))
 (segment (start 162.926 99.71) (end 163.89 99.71) (width 0.25) (layer "F.Cu") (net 22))
 (segment (start 160.1 104.07) (end 162.8 106.77) (width 0.25) (layer "F.Cu") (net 22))
 (segment (start 162.6 86.36) (end 164.67 86.36) (width 0.25) (layer "F.Cu") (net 22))
 (segment (start 159.8 100.838) (end 160.1 101.138) (width 0.25) (layer "F.Cu") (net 22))
 (segment (start 161.798 100.838) (end 162.926 99.71) (width 0.25) (layer "F.Cu") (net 22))
 (via (at 159.8 100.838) (size 0.8) (drill 0.4) (layers "F.Cu" "B.Cu") (free yes) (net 22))
 (via (at 162.6 86.36) (size 0.8) (drill 0.4) (layers "F.Cu" "B.Cu") (free yes) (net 22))
 (segment (start 160.115 100.523) (end 159.8 100.838) (width 0.25) (layer "B.Cu") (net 22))
 (segment (start 160.115 88.845) (end 160.115 100.523) (width 0.25) (layer "B.Cu") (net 22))
 (segment (start 162.6 86.36) (end 160.115 88.845) (width 0.25) (layer "B.Cu") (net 22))
 (segment (start 163.576 80.01) (end 164.67 80.01) (width 0.25) (layer "F.Cu") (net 27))
 (segment (start 160.3745 83.2115) (end 163.576 80.01) (width 0.25) (layer "F.Cu") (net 27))
 (segment (start 160.3745 83.312) (end 160.3745 83.2115) (width 0.25) (layer "F.Cu") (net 27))
 (via (at 160.3745 83.312) (size 0.8) (drill 0.4) (layers "F.Cu" "B.Cu") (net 27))
 (segment (start 157.575 104.975) (end 158.07 105.47) (width 0.25) (layer "B.Cu") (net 27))
 (segment (start 158.496 85.09) (end 158.496 96.256695) (width 0.25) (layer "B.Cu") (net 27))
 (segment (start 157.575 97.177695) (end 157.575 104.975) (width 0.25) (layer "B.Cu") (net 27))
 (segment (start 158.496 96.256695) (end 157.575 97.177695) (width 0.25) (layer "B.Cu") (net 27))
 (segment (start 158.07 105.47) (end 158.4 105.47) (width 0.25) (layer "B.Cu") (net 27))
 (segment (start 160.3745 83.312) (end 160.274 83.312) (width 0.25) (layer "B.Cu") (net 27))
 (segment (start 160.274 83.312) (end 158.496 85.09) (width 0.25) (layer "B.Cu") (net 27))
 (segment (start 157.951 79.982305) (end 156.2 78.231305) (width 0.25) (layer "B.Cu") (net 31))
 (segment (start 158.4 106.74) (end 158.243604 106.74) (width 0.25) (layer "B.Cu") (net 31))
 (segment (start 156.2 77.26) (end 152.6 73.66) (width 0.25) (layer "B.Cu") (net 31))
 (segment (start 157.125 96.991299) (end 157.951 96.165299) (width 0.25) (layer "B.Cu") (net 31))
 (segment (start 157.125 105.621396) (end 157.125 96.991299) (width 0.25) (layer "B.Cu") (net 31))
 (segment (start 158.243604 106.74) (end 157.125 105.621396) (width 0.25) (layer "B.Cu") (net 31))
 (segment (start 157.951 96.165299) (end 157.951 79.982305) (width 0.25) (layer "B.Cu") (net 31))
 (segment (start 156.2 78.231305) (end 156.2 77.26) (width 0.25) (layer "B.Cu") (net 31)))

